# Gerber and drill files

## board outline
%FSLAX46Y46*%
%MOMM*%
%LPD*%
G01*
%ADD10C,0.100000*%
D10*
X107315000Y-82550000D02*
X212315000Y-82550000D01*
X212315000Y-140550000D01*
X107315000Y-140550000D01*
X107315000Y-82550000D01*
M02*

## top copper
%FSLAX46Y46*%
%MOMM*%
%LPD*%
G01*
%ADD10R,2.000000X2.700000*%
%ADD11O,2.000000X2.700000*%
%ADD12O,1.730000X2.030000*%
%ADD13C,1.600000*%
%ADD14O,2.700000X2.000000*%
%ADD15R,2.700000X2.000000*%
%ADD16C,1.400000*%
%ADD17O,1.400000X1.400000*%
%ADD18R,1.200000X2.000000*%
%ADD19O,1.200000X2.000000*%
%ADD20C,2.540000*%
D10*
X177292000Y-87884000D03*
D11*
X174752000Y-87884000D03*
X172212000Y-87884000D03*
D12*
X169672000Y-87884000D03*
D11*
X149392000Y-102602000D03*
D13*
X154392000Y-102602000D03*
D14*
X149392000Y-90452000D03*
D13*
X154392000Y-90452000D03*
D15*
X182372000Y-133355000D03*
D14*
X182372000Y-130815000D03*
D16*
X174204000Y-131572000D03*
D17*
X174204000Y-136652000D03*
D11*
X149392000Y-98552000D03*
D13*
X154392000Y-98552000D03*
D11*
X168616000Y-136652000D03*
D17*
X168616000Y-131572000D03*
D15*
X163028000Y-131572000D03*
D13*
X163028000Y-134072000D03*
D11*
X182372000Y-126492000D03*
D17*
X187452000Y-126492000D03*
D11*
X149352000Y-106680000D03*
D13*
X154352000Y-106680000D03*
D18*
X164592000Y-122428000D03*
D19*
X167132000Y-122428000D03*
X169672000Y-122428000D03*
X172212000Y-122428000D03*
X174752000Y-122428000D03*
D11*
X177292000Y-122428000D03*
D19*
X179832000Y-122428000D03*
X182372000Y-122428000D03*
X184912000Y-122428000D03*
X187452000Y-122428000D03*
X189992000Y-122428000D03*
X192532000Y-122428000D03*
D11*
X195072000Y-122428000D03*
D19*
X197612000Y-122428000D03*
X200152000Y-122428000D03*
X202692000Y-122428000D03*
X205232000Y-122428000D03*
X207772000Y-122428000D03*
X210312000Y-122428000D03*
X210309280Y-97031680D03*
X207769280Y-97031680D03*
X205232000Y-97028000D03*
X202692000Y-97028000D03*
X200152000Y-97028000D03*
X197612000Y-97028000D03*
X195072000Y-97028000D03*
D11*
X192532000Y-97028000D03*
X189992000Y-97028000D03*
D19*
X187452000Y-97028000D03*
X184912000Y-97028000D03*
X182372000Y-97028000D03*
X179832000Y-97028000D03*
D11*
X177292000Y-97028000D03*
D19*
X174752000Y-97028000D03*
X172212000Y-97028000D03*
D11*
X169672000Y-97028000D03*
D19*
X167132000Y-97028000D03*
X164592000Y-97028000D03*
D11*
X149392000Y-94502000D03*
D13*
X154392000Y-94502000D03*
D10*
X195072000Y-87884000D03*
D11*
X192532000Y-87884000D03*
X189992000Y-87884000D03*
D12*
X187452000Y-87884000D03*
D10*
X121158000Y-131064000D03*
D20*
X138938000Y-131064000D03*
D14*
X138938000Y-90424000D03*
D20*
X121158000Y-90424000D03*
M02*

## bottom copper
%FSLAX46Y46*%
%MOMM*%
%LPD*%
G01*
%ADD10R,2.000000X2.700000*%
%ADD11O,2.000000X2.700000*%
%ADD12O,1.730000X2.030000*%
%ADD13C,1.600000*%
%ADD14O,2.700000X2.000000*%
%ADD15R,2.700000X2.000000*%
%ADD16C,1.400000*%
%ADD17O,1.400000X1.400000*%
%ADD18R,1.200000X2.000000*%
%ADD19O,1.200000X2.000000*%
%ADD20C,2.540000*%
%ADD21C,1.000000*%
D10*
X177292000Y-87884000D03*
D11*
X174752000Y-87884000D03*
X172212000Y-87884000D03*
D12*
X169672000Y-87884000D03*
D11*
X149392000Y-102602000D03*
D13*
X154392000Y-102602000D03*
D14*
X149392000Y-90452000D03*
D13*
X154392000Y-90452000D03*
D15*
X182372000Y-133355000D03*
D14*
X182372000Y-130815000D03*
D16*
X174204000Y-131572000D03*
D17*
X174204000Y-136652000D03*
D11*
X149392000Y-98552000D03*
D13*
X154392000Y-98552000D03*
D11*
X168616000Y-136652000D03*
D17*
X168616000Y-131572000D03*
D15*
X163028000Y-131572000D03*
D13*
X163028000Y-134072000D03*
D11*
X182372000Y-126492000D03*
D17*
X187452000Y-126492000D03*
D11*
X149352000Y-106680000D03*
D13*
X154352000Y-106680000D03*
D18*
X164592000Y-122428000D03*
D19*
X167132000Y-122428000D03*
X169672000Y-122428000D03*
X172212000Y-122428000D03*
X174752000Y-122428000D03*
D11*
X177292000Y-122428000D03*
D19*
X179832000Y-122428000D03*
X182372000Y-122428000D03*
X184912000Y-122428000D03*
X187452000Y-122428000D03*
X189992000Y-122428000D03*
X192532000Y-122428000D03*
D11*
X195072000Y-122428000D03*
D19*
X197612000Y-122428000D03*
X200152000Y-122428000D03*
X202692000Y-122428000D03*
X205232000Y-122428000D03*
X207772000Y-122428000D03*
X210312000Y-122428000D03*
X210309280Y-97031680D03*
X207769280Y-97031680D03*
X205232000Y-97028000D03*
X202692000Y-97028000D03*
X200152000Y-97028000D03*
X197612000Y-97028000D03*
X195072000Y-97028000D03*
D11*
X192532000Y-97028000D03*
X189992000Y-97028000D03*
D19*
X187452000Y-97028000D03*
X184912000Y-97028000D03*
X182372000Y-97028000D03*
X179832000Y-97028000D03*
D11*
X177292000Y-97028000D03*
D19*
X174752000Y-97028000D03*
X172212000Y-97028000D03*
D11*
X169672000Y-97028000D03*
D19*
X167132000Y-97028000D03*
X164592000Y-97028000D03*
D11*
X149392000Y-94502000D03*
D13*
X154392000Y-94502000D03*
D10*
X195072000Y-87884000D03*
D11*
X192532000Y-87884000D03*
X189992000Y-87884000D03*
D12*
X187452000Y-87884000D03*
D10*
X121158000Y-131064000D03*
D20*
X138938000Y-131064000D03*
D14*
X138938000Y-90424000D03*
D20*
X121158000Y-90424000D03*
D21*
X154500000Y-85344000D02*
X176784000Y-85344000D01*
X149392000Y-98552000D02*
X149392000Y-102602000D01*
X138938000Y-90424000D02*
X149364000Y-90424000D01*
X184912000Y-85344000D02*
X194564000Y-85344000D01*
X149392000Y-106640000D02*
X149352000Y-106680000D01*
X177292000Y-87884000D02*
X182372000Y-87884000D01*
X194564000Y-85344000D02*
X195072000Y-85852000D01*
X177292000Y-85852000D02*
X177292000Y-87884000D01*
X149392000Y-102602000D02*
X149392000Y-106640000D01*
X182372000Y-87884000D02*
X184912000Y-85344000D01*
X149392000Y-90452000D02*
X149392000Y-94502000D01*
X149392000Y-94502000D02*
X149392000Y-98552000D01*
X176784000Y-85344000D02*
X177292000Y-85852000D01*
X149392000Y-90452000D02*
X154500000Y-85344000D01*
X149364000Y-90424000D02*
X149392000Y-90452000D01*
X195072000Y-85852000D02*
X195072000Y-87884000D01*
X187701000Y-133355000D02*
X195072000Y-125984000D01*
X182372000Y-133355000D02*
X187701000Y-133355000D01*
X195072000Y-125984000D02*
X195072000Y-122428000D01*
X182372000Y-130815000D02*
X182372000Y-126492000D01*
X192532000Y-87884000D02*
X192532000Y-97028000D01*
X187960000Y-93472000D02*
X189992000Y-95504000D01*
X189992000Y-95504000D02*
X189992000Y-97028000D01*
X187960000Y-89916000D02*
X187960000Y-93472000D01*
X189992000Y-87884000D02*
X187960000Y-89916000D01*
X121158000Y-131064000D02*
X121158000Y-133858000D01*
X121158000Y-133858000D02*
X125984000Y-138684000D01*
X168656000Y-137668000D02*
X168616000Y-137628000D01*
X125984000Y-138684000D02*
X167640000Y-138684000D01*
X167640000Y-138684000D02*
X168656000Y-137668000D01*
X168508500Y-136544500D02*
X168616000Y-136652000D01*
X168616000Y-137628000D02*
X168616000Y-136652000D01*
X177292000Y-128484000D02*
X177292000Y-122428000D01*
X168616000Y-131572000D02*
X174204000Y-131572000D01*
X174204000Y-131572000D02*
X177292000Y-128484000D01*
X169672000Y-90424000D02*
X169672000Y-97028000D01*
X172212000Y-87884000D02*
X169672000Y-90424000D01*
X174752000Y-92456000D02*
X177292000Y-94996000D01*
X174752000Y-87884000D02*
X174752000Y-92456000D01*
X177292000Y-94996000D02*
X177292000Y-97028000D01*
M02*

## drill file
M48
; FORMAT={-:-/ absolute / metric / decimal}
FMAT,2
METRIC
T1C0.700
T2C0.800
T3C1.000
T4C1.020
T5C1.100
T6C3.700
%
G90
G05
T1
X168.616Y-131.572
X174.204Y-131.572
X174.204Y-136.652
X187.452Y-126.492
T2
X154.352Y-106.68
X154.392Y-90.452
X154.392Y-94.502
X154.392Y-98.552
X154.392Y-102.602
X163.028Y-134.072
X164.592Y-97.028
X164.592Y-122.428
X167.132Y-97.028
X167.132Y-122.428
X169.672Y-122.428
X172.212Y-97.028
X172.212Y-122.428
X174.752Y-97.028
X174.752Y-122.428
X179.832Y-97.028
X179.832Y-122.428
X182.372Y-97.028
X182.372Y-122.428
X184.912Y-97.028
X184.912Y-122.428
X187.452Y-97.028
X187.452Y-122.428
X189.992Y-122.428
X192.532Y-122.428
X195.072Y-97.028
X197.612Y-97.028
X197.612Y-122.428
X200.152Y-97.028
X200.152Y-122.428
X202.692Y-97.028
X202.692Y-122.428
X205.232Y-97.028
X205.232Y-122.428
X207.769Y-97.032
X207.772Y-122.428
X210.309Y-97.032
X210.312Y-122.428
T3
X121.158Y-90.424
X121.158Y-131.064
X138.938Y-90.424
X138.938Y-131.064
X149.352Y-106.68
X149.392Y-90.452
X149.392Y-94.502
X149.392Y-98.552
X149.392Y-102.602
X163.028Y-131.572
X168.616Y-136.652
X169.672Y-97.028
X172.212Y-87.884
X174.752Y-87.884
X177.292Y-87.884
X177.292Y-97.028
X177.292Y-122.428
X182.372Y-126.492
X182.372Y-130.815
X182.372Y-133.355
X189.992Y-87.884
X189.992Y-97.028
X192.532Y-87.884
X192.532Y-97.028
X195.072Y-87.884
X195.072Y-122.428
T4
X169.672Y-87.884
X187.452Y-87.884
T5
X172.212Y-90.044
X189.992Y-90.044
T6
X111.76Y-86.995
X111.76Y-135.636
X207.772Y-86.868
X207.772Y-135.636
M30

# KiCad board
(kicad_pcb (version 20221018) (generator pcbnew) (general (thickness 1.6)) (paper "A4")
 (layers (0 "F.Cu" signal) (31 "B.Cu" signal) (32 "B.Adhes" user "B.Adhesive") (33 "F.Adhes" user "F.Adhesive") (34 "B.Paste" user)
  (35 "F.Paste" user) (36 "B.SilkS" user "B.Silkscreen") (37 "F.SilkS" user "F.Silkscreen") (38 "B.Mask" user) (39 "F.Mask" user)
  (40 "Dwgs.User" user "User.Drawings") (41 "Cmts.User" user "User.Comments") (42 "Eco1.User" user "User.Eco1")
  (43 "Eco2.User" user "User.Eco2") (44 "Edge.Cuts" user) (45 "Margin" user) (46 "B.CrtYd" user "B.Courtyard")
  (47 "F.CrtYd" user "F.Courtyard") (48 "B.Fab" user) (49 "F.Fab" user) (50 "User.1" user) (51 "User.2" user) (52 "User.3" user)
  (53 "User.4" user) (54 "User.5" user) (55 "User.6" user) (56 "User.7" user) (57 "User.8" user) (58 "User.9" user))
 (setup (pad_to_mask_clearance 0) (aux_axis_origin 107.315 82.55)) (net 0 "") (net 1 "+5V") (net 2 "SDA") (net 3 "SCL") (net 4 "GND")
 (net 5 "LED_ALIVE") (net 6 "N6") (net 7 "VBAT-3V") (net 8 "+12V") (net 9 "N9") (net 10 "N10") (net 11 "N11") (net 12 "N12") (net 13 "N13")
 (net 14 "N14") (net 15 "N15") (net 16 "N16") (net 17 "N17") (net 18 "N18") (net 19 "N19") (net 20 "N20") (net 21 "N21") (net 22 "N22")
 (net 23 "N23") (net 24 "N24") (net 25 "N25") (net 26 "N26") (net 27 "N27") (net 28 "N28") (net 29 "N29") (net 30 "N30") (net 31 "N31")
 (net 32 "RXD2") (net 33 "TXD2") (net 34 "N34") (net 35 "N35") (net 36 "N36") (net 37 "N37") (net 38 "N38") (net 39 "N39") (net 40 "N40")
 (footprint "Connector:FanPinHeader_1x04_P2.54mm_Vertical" (layer "F.Cu") (at 177.292 87.884 180)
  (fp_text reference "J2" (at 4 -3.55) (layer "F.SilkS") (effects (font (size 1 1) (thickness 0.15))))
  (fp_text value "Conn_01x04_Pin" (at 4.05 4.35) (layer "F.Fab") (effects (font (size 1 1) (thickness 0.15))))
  (pad "" np_thru_hole circle (at 5.08 -2.16 270) (size 1.1 1.1) (drill 1.1) (layers "*.Cu" "*.Mask"))
  (pad "1" thru_hole rect (at 0 0 270) (size 2.7 2) (drill 1) (layers "*.Cu" "*.Mask") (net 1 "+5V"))
  (pad "2" thru_hole oval (at 2.54 0 90) (size 2.7 2) (drill 1) (layers "*.Cu" "*.Mask") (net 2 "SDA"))
  (pad "3" thru_hole oval (at 5.08 0 90) (size 2.7 2) (drill 1) (layers "*.Cu" "*.Mask") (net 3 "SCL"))
  (pad "4" thru_hole oval (at 7.62 0 270) (size 2.03 1.73) (drill 1.02) (layers "*.Cu" "*.Mask") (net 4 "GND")))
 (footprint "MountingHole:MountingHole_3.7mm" (layer "F.Cu") (at 207.772 86.868)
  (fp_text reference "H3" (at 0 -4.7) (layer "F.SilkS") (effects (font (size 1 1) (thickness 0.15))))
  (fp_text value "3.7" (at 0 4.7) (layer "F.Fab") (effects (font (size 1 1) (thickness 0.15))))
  (pad "" np_thru_hole circle (at 0 0) (size 3.7 3.7) (drill 3.7) (layers "*.Cu" "*.Mask")))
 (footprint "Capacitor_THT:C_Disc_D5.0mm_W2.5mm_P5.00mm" (layer "F.Cu") (at 149.392 102.602)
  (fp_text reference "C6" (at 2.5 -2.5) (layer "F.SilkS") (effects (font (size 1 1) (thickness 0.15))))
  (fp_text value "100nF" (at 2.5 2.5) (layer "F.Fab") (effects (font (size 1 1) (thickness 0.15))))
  (pad "1" thru_hole oval (at 0 0) (size 2 2.7) (drill 1) (layers "*.Cu" "*.Mask") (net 1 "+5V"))
  (pad "2" thru_hole circle (at 5 0) (size 1.6 1.6) (drill 0.8) (layers "*.Cu" "*.Mask") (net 4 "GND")))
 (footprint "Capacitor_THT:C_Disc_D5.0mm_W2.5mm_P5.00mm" (layer "F.Cu") (at 149.392 90.452)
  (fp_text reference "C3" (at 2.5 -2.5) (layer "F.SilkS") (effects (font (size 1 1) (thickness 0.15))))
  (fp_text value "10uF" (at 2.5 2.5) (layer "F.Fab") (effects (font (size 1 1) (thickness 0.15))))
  (pad "1" thru_hole oval (at 0 0) (size 2.7 2) (drill 1) (layers "*.Cu" "*.Mask") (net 1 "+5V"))
  (pad "2" thru_hole circle (at 5 0) (size 1.6 1.6) (drill 0.8) (layers "*.Cu" "*.Mask") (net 4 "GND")))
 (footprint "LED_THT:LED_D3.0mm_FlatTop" (layer "F.Cu") (at 182.372 133.355 90)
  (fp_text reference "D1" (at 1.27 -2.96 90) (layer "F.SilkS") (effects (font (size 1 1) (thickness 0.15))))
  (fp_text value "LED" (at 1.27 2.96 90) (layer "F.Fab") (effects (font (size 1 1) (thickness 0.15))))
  (pad "1" thru_hole rect (at 0 0 180) (size 2.7 2) (drill 1) (layers "*.Cu" "*.Mask") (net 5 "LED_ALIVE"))
  (pad "2" thru_hole oval (at 2.54 0 90) (size 2 2.7) (drill 1) (layers "*.Cu" "*.Mask") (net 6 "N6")))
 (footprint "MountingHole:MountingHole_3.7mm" (layer "F.Cu") (at 111.76 135.636)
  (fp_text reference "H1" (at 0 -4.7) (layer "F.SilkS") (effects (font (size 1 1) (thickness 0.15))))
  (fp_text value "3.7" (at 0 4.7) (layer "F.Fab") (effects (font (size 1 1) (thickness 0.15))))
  (pad "" np_thru_hole circle (at 0 0) (size 3.7 3.7) (drill 3.7) (layers "*.Cu" "*.Mask")))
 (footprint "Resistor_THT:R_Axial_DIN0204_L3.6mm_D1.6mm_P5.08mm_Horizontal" (layer "F.Cu") (at 174.204 131.572 -90)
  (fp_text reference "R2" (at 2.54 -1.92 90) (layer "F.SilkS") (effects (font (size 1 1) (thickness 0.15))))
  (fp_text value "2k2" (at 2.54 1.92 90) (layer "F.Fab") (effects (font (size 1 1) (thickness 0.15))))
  (pad "1" thru_hole circle (at 0 0 270) (size 1.4 1.4) (drill 0.7) (layers "*.Cu" "*.Mask") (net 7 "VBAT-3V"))
  (pad "2" thru_hole oval (at 5.08 0 270) (size 1.4 1.4) (drill 0.7) (layers "*.Cu" "*.Mask") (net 4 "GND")))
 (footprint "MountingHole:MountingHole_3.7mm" (layer "F.Cu") (at 207.772 135.636)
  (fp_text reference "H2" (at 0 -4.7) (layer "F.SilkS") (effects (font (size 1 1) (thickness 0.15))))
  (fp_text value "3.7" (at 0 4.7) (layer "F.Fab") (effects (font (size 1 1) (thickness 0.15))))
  (pad "" np_thru_hole circle (at 0 0) (size 3.7 3.7) (drill 3.7) (layers "*.Cu" "*.Mask")))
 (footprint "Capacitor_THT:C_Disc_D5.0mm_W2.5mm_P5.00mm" (layer "F.Cu") (at 149.392 98.552)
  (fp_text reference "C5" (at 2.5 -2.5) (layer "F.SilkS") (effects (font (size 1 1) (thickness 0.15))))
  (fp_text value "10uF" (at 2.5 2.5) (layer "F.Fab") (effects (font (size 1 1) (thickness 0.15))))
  (pad "1" thru_hole oval (at 0 0) (size 2 2.7) (drill 1) (layers "*.Cu" "*.Mask") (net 1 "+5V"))
  (pad "2" thru_hole circle (at 5 0) (size 1.6 1.6) (drill 0.8) (layers "*.Cu" "*.Mask") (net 4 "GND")))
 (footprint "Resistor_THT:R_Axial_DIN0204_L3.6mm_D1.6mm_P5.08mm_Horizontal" (layer "F.Cu") (at 168.616 136.652 90)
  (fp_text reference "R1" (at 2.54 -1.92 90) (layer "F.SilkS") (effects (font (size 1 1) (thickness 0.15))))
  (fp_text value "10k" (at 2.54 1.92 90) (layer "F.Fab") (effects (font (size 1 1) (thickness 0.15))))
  (pad "1" thru_hole oval (at 0 0 90) (size 2.7 2) (drill 1) (layers "*.Cu" "*.Mask") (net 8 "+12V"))
  (pad "2" thru_hole oval (at 5.08 0 90) (size 1.4 1.4) (drill 0.7) (layers "*.Cu" "*.Mask") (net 7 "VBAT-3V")))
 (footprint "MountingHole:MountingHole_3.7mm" (layer "F.Cu") (at 111.76 86.995)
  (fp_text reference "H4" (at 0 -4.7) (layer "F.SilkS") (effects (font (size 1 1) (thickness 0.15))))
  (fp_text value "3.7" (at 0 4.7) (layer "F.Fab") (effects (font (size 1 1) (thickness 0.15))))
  (pad "" np_thru_hole circle (at 0 0) (size 3.7 3.7) (drill 3.7) (layers "*.Cu" "*.Mask")))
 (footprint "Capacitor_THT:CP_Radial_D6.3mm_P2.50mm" (layer "F.Cu") (at 163.028 131.572 -90)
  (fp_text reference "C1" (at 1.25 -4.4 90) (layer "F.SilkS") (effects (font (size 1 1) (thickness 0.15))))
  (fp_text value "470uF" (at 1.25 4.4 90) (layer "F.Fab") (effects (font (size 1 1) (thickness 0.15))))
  (pad "1" thru_hole rect (at 0 0) (size 2.7 2) (drill 1) (layers "*.Cu" "*.Mask") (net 1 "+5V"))
  (pad "2" thru_hole circle (at 2.5 0 270) (size 1.6 1.6) (drill 0.8) (layers "*.Cu" "*.Mask") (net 4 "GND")))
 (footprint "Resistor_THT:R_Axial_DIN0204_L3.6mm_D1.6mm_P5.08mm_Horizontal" (layer "F.Cu") (at 182.372 126.492)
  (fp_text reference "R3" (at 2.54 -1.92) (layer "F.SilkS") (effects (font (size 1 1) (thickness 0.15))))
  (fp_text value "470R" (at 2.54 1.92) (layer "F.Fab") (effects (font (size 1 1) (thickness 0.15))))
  (pad "1" thru_hole oval (at 0 0) (size 2 2.7) (drill 1) (layers "*.Cu" "*.Mask") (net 6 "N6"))
  (pad "2" thru_hole oval (at 5.08 0) (size 1.4 1.4) (drill 0.7) (layers "*.Cu" "*.Mask") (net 4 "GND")))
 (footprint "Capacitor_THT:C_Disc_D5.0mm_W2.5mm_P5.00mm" (layer "F.Cu") (at 149.352 106.68)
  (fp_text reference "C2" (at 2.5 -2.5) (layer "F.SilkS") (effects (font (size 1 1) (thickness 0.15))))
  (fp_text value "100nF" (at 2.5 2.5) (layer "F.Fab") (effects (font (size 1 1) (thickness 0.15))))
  (pad "1" thru_hole oval (at 0 0) (size 2 2.7) (drill 1) (layers "*.Cu" "*.Mask") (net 1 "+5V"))
  (pad "2" thru_hole circle (at 5 0) (size 1.6 1.6) (drill 0.8) (layers "*.Cu" "*.Mask") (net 4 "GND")))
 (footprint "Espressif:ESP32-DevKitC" (layer "F.Cu") (at 164.592 122.428 90)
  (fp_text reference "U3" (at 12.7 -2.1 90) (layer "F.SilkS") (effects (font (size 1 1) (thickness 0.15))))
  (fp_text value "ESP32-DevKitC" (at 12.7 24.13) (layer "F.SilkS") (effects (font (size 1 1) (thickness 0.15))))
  (pad "1" thru_hole rect (at 0 0) (size 1.2 2) (drill 0.8) (layers "*.Cu" "*.Mask") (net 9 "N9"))
  (pad "2" thru_hole oval (at 0 2.54) (size 1.2 2) (drill 0.8) (layers "*.Cu" "*.Mask") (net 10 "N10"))
  (pad "3" thru_hole oval (at 0 5.08) (size 1.2 2) (drill 0.8) (layers "*.Cu" "*.Mask") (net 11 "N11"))
  (pad "4" thru_hole oval (at 0 7.62) (size 1.2 2) (drill 0.8) (layers "*.Cu" "*.Mask") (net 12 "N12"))
  (pad "5" thru_hole oval (at 0 10.16) (size 1.2 2) (drill 0.8) (layers "*.Cu" "*.Mask") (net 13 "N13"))
  (pad "6" thru_hole oval (at 0 12.7) (size 2 2.7) (drill 1) (layers "*.Cu" "*.Mask") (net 7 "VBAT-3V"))
  (pad "7" thru_hole oval (at 0 15.24) (size 1.2 2) (drill 0.8) (layers "*.Cu" "*.Mask") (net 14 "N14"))
  (pad "8" thru_hole oval (at 0 17.78) (size 1.2 2) (drill 0.8) (layers "*.Cu" "*.Mask") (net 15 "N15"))
  (pad "9" thru_hole oval (at 0 20.32) (size 1.2 2) (drill 0.8) (layers "*.Cu" "*.Mask") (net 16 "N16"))
  (pad "10" thru_hole oval (at 0 22.86) (size 1.2 2) (drill 0.8) (layers "*.Cu" "*.Mask") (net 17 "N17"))
  (pad "11" thru_hole oval (at 0 25.4) (size 1.2 2) (drill 0.8) (layers "*.Cu" "*.Mask") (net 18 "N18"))
  (pad "12" thru_hole oval (at 0 27.94) (size 1.2 2) (drill 0.8) (layers "*.Cu" "*.Mask") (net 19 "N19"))
  (pad "13" thru_hole oval (at 0 30.48) (size 2 2.7) (drill 1) (layers "*.Cu" "*.Mask") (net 5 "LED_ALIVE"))
  (pad "14" thru_hole oval (at 0 33.02) (size 1.2 2) (drill 0.8) (layers "*.Cu" "*.Mask") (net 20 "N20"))
  (pad "15" thru_hole oval (at 0 35.56) (size 1.2 2) (drill 0.8) (layers "*.Cu" "*.Mask") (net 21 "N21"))
  (pad "16" thru_hole oval (at 0 38.1) (size 1.2 2) (drill 0.8) (layers "*.Cu" "*.Mask") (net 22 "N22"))
  (pad "17" thru_hole oval (at 0 40.64) (size 1.2 2) (drill 0.8) (layers "*.Cu" "*.Mask") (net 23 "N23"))
  (pad "18" thru_hole oval (at 0 43.18) (size 1.2 2) (drill 0.8) (layers "*.Cu" "*.Mask") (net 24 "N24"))
  (pad "19" thru_hole oval (at 0 45.72) (size 1.2 2) (drill 0.8) (layers "*.Cu" "*.Mask") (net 1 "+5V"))
  (pad "20" thru_hole oval (at 25.39632 45.71728) (size 1.2 2) (drill 0.8) (layers "*.Cu" "*.Mask") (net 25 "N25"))
  (pad "21" thru_hole oval (at 25.39632 43.17728) (size 1.2 2) (drill 0.8) (layers "*.Cu" "*.Mask") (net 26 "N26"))
  (pad "22" thru_hole oval (at 25.4 40.64) (size 1.2 2) (drill 0.8) (layers "*.Cu" "*.Mask") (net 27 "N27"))
  (pad "23" thru_hole oval (at 25.4 38.1) (size 1.2 2) (drill 0.8) (layers "*.Cu" "*.Mask") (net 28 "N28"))
  (pad "24" thru_hole oval (at 25.4 35.56) (size 1.2 2) (drill 0.8) (layers "*.Cu" "*.Mask") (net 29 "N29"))
  (pad "25" thru_hole oval (at 25.4 33.02) (size 1.2 2) (drill 0.8) (layers "*.Cu" "*.Mask") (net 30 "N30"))
  (pad "26" thru_hole oval (at 25.4 30.48) (size 1.2 2) (drill 0.8) (layers "*.Cu" "*.Mask") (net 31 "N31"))
  (pad "27" thru_hole oval (at 25.4 27.94) (size 2 2.7) (drill 1) (layers "*.Cu" "*.Mask") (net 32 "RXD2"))
  (pad "28" thru_hole oval (at 25.4 25.4) (size 2 2.7) (drill 1) (layers "*.Cu" "*.Mask") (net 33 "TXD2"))
  (pad "29" thru_hole oval (at 25.4 22.86) (size 1.2 2) (drill 0.8) (layers "*.Cu" "*.Mask") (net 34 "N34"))
  (pad "30" thru_hole oval (at 25.4 20.32) (size 1.2 2) (drill 0.8) (layers "*.Cu" "*.Mask") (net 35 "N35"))
  (pad "31" thru_hole oval (at 25.4 17.78) (size 1.2 2) (drill 0.8) (layers "*.Cu" "*.Mask") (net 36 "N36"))
  (pad "32" thru_hole oval (at 25.4 15.24) (size 1.2 2) (drill 0.8) (layers "*.Cu" "*.Mask") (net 4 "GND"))
  (pad "33" thru_hole oval (at 25.4 12.7) (size 2 2.7) (drill 1) (layers "*.Cu" "*.Mask") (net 2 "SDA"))
  (pad "34" thru_hole oval (at 25.4 10.16) (size 1.2 2) (drill 0.8) (layers "*.Cu" "*.Mask") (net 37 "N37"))
  (pad "35" thru_hole oval (at 25.4 7.62) (size 1.2 2) (drill 0.8) (layers "*.Cu" "*.Mask") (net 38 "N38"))
  (pad "36" thru_hole oval (at 25.4 5.08) (size 2 2.7) (drill 1) (layers "*.Cu" "*.Mask") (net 3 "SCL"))
  (pad "37" thru_hole oval (at 25.4 2.54) (size 1.2 2) (drill 0.8) (layers "*.Cu" "*.Mask") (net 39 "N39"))
  (pad "38" thru_hole oval (at 25.4 0) (size 1.2 2) (drill 0.8) (layers "*.Cu" "*.Mask") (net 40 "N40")))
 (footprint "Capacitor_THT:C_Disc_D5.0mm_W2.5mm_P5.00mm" (layer "F.Cu") (at 149.392 94.502)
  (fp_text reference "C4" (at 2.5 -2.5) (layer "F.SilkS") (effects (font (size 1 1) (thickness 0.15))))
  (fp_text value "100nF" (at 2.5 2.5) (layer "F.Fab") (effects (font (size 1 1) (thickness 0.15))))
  (pad "1" thru_hole oval (at 0 0) (size 2 2.7) (drill 1) (layers "*.Cu" "*.Mask") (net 1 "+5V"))
  (pad "2" thru_hole circle (at 5 0) (size 1.6 1.6) (drill 0.8) (layers "*.Cu" "*.Mask") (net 4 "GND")))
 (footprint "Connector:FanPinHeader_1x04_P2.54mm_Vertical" (layer "F.Cu") (at 195.072 87.884 180)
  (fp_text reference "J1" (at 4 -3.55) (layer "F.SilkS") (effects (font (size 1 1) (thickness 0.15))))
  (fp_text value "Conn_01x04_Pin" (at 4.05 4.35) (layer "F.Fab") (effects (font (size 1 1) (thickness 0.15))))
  (pad "" np_thru_hole circle (at 5.08 -2.16 270) (size 1.1 1.1) (drill 1.1) (layers "*.Cu" "*.Mask"))
  (pad "1" thru_hole rect (at 0 0 270) (size 2.7 2) (drill 1) (layers "*.Cu" "*.Mask") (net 1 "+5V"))
  (pad "2" thru_hole oval (at 2.54 0 90) (size 2.7 2) (drill 1) (layers "*.Cu" "*.Mask") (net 32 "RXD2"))
  (pad "3" thru_hole oval (at 5.08 0 90) (size 2.7 2) (drill 1) (layers "*.Cu" "*.Mask") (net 33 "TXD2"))
  (pad "4" thru_hole oval (at 7.62 0 270) (size 2.03 1.73) (drill 1.02) (layers "*.Cu" "*.Mask") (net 4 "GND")))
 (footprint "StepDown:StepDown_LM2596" (layer "F.Cu") (at 121.158 131.064 90)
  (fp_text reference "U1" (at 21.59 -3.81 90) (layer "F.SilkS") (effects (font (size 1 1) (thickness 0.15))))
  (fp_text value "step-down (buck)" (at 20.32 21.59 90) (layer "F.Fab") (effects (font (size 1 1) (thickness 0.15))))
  (pad "1" thru_hole rect (at 0 0 180) (size 2 2.7) (drill 1) (layers "*.Cu" "*.Mask") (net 8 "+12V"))
  (pad "2" thru_hole circle (at 0 17.78 90) (size 2.54 2.54) (drill 1) (layers "*.Cu" "*.Mask") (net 4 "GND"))
  (pad "3" thru_hole oval (at 40.64 17.78 90) (size 2 2.7) (drill 1) (layers "*.Cu" "*.Mask") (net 1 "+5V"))
  (pad "4" thru_hole circle (at 40.64 0 90) (size 2.54 2.54) (drill 1) (layers "*.Cu" "*.Mask")))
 (gr_rect (start 107.315 82.55) (end 212.315 140.55) (stroke (width 0.1) (type default)) (fill none) (layer "Edge.Cuts"))
 (segment (start 154.5 85.344) (end 176.784 85.344) (width 1) (layer "B.Cu") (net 1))
 (segment (start 149.392 98.552) (end 149.392 102.602) (width 1) (layer "B.Cu") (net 1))
 (segment (start 138.938 90.424) (end 149.364 90.424) (width 1) (layer "B.Cu") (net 1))
 (segment (start 184.912 85.344) (end 194.564 85.344) (width 1) (layer "B.Cu") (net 1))
 (segment (start 149.392 106.64) (end 149.352 106.68) (width 1) (layer "B.Cu") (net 1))
 (segment (start 177.292 87.884) (end 182.372 87.884) (width 1) (layer "B.Cu") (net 1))
 (segment (start 194.564 85.344) (end 195.072 85.852) (width 1) (layer "B.Cu") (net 1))
 (segment (start 177.292 85.852) (end 177.292 87.884) (width 1) (layer "B.Cu") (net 1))
 (segment (start 149.392 102.602) (end 149.392 106.64) (width 1) (layer "B.Cu") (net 1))
 (segment (start 182.372 87.884) (end 184.912 85.344) (width 1) (layer "B.Cu") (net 1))
 (segment (start 149.392 90.452) (end 149.392 94.502) (width 1) (layer "B.Cu") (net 1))
 (segment (start 149.392 94.502) (end 149.392 98.552) (width 1) (layer "B.Cu") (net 1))
 (segment (start 176.784 85.344) (end 177.292 85.852) (width 1) (layer "B.Cu") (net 1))
 (segment (start 149.392 90.452) (end 154.5 85.344) (width 1) (layer "B.Cu") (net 1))
 (segment (start 149.364 90.424) (end 149.392 90.452) (width 1) (layer "B.Cu") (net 1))
 (segment (start 195.072 85.852) (end 195.072 87.884) (width 1) (layer "B.Cu") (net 1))
 (segment (start 187.701 133.355) (end 195.072 125.984) (width 1) (layer "B.Cu") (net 5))
 (segment (start 182.372 133.355) (end 187.701 133.355) (width 1) (layer "B.Cu") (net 5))
 (segment (start 195.072 125.984) (end 195.072 122.428) (width 1) (layer "B.Cu") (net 5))
 (segment (start 182.372 130.815) (end 182.372 126.492) (width 1) (layer "B.Cu") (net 6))
 (segment (start 192.532 87.884) (end 192.532 97.028) (width 1) (layer "B.Cu") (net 32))
 (segment (start 187.96 93.472) (end 189.992 95.504) (width 1) (layer "B.Cu") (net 33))
 (segment (start 189.992 95.504) (end 189.992 97.028) (width 1) (layer "B.Cu") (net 33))
 (segment (start 187.96 89.916) (end 187.96 93.472) (width 1) (layer "B.Cu") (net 33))
 (segment (start 189.992 87.884) (end 187.96 89.916) (width 1) (layer "B.Cu") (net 33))
 (segment (start 121.158 131.064) (end 121.158 133.858) (width 1) (layer "B.Cu") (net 8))
 (segment (start 121.158 133.858) (end 125.984 138.684) (width 1) (layer "B.Cu") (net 8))
 (segment (start 168.656 137.668) (end 168.616 137.628) (width 1) (layer "B.Cu") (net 8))
 (segment (start 125.984 138.684) (end 167.64 138.684) (width 1) (layer "B.Cu") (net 8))
 (segment (start 167.64 138.684) (end 168.656 137.668) (width 1) (layer "B.Cu") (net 8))
 (segment (start 168.5085 136.5445) (end 168.616 136.652) (width 1) (layer "B.Cu") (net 8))
 (segment (start 168.616 137.628) (end 168.616 136.652) (width 1) (layer "B.Cu") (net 8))
 (segment (start 177.292 128.484) (end 177.292 122.428) (width 1) (layer "B.Cu") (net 7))
 (segment (start 168.616 131.572) (end 174.204 131.572) (width 1) (layer "B.Cu") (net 7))
 (segment (start 174.204 131.572) (end 177.292 128.484) (width 1) (layer "B.Cu") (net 7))
 (segment (start 169.672 90.424) (end 169.672 97.028) (width 1) (layer "B.Cu") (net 3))
 (segment (start 172.212 87.884) (end 169.672 90.424) (width 1) (layer "B.Cu") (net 3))
 (segment (start 174.752 92.456) (end 177.292 94.996) (width 1) (layer "B.Cu") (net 2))
 (segment (start 174.752 87.884) (end 174.752 92.456) (width 1) (layer "B.Cu") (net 2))
 (segment (start 177.292 94.996) (end 177.292 97.028) (width 1) (layer "B.Cu") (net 2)))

